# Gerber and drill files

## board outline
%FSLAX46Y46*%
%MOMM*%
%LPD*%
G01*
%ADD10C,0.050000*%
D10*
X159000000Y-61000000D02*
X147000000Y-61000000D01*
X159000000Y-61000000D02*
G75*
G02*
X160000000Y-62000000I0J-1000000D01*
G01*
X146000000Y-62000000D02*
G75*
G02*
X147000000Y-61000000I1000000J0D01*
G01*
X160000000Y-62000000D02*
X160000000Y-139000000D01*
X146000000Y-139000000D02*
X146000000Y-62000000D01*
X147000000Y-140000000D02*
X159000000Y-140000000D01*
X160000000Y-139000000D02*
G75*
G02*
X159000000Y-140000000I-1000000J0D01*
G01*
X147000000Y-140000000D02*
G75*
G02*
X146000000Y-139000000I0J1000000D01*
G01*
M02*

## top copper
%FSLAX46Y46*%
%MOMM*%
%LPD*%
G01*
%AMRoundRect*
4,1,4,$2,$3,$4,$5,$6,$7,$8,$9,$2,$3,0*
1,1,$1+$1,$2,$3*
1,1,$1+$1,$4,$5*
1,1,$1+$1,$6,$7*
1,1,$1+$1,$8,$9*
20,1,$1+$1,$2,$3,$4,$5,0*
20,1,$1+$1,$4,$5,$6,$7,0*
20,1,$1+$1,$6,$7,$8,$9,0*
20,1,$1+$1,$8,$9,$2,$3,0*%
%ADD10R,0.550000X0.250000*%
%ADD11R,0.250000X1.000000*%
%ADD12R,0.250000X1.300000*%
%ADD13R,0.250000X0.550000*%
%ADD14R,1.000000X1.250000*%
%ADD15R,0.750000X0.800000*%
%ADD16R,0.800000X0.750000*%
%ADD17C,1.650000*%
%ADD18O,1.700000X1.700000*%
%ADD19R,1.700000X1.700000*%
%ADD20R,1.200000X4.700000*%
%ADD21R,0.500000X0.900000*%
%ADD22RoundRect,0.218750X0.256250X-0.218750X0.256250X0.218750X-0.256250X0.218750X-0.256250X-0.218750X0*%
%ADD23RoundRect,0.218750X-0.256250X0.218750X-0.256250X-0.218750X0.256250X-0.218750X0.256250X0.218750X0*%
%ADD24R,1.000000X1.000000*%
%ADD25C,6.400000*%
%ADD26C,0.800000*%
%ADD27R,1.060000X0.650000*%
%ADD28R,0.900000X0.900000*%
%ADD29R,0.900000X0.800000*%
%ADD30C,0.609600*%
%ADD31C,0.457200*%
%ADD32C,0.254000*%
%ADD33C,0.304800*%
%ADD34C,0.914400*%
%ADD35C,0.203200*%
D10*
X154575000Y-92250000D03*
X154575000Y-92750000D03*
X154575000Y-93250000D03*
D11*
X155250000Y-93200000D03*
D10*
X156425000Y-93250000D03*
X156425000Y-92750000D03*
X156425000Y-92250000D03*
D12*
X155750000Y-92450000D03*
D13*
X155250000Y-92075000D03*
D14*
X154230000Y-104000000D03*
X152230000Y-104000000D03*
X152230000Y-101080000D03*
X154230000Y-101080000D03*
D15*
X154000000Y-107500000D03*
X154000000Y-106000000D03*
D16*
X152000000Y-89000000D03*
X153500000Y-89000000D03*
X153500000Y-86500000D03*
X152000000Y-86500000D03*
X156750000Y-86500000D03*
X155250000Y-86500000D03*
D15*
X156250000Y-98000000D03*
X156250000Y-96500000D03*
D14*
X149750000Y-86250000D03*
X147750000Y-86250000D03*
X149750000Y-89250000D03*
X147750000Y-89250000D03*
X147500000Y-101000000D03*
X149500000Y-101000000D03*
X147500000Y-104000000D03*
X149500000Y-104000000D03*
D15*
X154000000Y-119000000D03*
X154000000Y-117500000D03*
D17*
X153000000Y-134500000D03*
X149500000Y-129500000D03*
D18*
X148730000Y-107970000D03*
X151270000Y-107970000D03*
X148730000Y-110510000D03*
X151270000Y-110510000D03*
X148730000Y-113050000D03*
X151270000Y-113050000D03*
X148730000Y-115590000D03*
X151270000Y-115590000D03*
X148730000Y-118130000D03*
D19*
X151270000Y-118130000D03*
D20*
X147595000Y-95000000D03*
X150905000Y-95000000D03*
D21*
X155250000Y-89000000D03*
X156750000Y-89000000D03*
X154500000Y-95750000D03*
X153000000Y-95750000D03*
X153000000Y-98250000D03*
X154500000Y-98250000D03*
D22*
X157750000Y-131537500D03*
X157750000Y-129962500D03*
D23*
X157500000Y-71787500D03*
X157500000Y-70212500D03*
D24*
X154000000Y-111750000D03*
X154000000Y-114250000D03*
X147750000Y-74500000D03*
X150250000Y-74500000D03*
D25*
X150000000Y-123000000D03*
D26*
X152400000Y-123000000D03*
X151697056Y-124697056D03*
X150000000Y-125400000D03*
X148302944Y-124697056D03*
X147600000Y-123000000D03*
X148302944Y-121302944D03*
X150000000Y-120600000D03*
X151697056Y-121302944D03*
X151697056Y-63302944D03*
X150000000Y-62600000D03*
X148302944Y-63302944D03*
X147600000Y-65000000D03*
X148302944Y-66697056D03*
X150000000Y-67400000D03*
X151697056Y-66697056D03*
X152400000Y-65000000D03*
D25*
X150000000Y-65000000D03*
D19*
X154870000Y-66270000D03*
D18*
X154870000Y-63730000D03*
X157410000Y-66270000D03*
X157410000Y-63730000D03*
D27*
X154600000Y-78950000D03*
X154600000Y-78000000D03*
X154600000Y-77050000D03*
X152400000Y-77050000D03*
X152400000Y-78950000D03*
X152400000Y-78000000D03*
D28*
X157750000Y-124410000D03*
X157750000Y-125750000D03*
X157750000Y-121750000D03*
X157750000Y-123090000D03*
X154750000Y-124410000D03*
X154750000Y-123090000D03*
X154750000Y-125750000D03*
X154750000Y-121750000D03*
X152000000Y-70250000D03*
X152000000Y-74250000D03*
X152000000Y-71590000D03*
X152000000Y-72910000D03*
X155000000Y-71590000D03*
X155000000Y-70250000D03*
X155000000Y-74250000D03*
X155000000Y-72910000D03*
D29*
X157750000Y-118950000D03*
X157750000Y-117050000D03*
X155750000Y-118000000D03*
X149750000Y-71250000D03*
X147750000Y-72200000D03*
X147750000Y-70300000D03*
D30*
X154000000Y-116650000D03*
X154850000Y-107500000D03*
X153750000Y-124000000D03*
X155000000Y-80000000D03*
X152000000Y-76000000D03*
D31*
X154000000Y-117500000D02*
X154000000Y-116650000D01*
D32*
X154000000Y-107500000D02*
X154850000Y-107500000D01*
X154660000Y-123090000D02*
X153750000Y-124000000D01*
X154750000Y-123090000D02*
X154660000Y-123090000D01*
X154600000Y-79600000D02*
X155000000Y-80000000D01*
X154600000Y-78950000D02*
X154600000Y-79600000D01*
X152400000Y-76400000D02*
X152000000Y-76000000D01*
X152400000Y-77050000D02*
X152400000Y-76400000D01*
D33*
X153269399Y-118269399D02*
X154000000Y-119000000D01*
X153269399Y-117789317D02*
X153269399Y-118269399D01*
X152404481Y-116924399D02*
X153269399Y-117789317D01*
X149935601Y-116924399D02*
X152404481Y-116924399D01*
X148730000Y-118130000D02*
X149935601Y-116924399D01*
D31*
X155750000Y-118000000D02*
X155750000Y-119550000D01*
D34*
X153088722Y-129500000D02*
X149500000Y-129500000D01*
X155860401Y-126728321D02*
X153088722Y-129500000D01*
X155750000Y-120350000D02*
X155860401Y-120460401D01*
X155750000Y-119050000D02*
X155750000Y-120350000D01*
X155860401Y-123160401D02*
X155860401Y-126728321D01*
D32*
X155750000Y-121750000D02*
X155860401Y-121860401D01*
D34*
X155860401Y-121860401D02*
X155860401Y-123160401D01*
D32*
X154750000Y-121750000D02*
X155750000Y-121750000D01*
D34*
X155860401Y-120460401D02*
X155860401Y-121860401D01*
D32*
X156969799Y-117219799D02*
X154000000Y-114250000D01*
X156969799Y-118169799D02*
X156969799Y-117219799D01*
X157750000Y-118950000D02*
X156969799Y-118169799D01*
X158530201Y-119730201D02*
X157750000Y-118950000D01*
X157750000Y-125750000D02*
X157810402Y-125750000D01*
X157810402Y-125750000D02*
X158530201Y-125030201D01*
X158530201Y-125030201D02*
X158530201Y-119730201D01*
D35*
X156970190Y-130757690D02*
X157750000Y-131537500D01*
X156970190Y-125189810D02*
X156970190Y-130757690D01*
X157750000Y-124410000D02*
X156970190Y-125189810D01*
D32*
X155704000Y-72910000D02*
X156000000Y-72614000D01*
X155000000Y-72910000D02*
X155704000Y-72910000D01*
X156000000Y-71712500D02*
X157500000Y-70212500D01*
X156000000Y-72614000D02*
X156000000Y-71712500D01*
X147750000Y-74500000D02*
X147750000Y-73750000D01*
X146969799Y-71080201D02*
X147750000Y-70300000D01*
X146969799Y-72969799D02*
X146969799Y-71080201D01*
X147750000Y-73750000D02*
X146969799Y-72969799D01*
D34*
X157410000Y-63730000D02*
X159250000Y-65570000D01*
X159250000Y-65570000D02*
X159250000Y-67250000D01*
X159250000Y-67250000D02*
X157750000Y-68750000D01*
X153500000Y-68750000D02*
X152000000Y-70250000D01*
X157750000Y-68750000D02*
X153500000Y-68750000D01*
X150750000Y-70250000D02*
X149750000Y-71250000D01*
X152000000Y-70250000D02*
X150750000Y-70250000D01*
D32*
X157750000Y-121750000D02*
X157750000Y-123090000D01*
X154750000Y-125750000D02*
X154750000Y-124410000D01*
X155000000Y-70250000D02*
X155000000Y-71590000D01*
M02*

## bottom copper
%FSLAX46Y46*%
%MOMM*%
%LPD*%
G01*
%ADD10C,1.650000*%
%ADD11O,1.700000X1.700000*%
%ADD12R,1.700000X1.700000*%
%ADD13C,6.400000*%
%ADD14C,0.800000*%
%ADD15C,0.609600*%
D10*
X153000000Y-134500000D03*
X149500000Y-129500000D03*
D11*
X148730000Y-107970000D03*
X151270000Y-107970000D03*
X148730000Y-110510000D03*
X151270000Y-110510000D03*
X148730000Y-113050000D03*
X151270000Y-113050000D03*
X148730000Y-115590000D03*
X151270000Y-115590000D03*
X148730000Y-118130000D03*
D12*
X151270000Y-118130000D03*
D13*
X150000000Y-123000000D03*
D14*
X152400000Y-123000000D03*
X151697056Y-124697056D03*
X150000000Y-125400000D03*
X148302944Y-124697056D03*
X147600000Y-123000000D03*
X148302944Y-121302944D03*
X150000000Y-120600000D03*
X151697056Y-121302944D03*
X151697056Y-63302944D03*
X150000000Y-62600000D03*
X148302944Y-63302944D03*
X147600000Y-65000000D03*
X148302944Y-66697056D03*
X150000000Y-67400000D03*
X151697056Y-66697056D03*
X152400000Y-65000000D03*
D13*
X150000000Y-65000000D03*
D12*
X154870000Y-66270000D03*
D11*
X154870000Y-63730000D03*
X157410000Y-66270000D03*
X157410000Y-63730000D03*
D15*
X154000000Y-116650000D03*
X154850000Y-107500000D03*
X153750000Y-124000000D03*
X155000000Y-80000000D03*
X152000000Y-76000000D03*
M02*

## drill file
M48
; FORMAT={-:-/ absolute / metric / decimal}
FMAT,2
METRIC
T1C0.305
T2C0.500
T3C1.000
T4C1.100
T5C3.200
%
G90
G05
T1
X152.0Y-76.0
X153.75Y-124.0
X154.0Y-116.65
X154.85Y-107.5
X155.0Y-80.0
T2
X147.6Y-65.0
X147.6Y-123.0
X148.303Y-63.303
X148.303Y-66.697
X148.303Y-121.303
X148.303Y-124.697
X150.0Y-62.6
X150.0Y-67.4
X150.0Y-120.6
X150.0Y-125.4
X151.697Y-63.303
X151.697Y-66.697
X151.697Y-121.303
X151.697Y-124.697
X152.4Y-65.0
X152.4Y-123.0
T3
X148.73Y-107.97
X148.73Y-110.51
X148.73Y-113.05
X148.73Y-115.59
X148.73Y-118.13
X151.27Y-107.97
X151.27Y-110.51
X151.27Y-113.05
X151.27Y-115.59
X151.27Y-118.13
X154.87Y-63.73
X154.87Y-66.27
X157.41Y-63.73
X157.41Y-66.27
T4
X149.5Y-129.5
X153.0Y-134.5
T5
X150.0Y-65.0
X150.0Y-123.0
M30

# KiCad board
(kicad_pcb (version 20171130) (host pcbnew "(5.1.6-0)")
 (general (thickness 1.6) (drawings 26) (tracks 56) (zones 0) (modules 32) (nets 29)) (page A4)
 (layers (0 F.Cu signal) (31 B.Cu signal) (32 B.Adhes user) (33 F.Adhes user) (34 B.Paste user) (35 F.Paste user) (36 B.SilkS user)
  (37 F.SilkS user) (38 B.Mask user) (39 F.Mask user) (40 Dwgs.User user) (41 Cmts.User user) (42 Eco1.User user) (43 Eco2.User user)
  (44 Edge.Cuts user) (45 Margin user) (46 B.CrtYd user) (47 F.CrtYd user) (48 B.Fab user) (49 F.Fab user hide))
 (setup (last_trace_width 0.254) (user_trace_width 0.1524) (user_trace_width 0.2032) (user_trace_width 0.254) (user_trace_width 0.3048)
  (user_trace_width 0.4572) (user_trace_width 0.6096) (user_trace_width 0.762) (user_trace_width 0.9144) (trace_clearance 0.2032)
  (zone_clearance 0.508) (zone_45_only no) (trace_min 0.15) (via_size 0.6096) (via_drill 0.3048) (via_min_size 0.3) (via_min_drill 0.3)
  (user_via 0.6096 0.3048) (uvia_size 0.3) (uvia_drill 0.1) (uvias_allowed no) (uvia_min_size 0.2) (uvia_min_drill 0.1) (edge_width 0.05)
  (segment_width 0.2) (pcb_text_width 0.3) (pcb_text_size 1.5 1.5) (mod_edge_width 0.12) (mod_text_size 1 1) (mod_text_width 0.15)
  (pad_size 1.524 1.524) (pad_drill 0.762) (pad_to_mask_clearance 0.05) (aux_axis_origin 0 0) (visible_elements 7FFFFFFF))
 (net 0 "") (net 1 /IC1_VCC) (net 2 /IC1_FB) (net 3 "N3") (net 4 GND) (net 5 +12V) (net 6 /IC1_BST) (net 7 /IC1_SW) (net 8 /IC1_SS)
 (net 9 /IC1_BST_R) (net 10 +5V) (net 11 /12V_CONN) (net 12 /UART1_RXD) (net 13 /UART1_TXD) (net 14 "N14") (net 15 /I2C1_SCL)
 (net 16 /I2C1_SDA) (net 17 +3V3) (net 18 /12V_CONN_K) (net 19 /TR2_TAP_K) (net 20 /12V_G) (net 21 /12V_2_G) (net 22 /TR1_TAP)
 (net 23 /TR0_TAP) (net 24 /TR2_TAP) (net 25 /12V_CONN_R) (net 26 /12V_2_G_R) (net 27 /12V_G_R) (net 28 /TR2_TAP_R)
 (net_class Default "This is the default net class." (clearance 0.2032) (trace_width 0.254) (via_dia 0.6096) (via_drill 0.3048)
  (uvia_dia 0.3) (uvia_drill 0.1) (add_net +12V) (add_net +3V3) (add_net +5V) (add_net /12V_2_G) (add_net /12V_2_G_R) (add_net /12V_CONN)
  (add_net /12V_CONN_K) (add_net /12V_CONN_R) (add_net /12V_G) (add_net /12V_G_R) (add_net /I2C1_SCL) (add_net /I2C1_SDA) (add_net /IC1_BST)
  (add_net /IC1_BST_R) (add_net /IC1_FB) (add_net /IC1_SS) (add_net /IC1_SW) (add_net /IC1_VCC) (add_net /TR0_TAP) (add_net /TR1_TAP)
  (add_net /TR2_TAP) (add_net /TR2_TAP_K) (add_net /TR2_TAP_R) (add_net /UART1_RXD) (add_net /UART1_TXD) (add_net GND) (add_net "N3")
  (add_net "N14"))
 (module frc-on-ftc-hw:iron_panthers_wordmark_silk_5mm (layer F.Cu) (at 157.5 108 90)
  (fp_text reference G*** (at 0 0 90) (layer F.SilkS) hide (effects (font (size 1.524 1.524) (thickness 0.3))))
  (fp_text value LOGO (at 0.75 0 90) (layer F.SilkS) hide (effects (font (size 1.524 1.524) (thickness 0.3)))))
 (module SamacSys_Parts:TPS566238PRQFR (layer F.Cu) (at 155.5 92.75)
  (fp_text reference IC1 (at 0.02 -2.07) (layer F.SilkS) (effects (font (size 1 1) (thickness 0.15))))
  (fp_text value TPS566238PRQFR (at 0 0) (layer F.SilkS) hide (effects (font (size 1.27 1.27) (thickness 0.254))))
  (pad 1 smd rect (at -0.925 -0.5 90) (size 0.25 0.55) (layers F.Cu F.Paste F.Mask) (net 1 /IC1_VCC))
  (pad 2 smd rect (at -0.925 0 90) (size 0.25 0.55) (layers F.Cu F.Paste F.Mask) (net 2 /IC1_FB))
  (pad 3 smd rect (at -0.925 0.5 90) (size 0.25 0.55) (layers F.Cu F.Paste F.Mask) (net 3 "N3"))
  (pad 4 smd rect (at -0.25 0.45) (size 0.25 1) (layers F.Cu F.Paste F.Mask) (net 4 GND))
  (pad 5 smd rect (at 0.925 0.5 90) (size 0.25 0.55) (layers F.Cu F.Paste F.Mask) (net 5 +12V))
  (pad 6 smd rect (at 0.925 0 90) (size 0.25 0.55) (layers F.Cu F.Paste F.Mask) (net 5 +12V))
  (pad 7 smd rect (at 0.925 -0.5 90) (size 0.25 0.55) (layers F.Cu F.Paste F.Mask) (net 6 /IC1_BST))
  (pad 8 smd rect (at 0.25 -0.3) (size 0.25 1.3) (layers F.Cu F.Paste F.Mask) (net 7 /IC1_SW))
  (pad 9 smd rect (at -0.25 -0.675) (size 0.25 0.55) (layers F.Cu F.Paste F.Mask) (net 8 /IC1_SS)))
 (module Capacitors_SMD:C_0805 (layer F.Cu) (at 153.23 104 180)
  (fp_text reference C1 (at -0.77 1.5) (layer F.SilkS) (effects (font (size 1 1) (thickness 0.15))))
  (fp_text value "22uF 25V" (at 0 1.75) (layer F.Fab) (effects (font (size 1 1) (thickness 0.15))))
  (pad 1 smd rect (at -1 0 180) (size 1 1.25) (layers F.Cu F.Paste F.Mask) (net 5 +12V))
  (pad 2 smd rect (at 1 0 180) (size 1 1.25) (layers F.Cu F.Paste F.Mask) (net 4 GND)))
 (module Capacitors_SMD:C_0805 (layer F.Cu) (at 153.23 101.08 180)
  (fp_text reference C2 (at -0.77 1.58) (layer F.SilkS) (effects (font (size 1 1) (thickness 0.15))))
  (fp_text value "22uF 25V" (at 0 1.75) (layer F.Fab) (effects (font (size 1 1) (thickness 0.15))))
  (pad 2 smd rect (at 1 0 180) (size 1 1.25) (layers F.Cu F.Paste F.Mask) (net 4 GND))
  (pad 1 smd rect (at -1 0 180) (size 1 1.25) (layers F.Cu F.Paste F.Mask) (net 5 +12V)))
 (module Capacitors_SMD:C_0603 (layer F.Cu) (at 154 106.75 270)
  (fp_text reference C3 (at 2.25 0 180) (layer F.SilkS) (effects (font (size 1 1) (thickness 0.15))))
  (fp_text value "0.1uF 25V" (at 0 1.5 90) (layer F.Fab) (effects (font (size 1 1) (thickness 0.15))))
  (pad 2 smd rect (at 0.75 0 270) (size 0.8 0.75) (layers F.Cu F.Paste F.Mask) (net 4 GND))
  (pad 1 smd rect (at -0.75 0 270) (size 0.8 0.75) (layers F.Cu F.Paste F.Mask) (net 5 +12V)))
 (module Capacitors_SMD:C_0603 (layer F.Cu) (at 152.75 89 180)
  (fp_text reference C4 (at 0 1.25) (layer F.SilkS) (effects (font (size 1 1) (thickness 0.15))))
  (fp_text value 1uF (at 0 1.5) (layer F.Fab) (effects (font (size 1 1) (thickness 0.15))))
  (pad 2 smd rect (at 0.75 0 180) (size 0.8 0.75) (layers F.Cu F.Paste F.Mask) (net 4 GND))
  (pad 1 smd rect (at -0.75 0 180) (size 0.8 0.75) (layers F.Cu F.Paste F.Mask) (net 1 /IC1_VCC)))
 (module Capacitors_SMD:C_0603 (layer F.Cu) (at 152.75 86.5 180)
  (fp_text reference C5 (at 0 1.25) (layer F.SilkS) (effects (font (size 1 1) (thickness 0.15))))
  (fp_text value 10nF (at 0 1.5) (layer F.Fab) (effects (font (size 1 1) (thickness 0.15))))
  (pad 1 smd rect (at -0.75 0 180) (size 0.8 0.75) (layers F.Cu F.Paste F.Mask) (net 8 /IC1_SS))
  (pad 2 smd rect (at 0.75 0 180) (size 0.8 0.75) (layers F.Cu F.Paste F.Mask) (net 4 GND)))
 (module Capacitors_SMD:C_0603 (layer F.Cu) (at 156 86.5)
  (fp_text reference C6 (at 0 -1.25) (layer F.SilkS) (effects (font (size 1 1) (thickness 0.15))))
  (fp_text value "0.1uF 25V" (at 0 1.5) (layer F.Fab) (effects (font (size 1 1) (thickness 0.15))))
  (pad 2 smd rect (at 0.75 0) (size 0.8 0.75) (layers F.Cu F.Paste F.Mask) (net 7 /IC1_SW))
  (pad 1 smd rect (at -0.75 0) (size 0.8 0.75) (layers F.Cu F.Paste F.Mask) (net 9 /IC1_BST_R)))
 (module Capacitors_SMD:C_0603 (layer F.Cu) (at 156.25 97.25 90)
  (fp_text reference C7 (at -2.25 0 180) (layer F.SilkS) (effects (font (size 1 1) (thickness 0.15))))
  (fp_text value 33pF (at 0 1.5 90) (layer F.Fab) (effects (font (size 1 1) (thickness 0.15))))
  (pad 1 smd rect (at -0.75 0 90) (size 0.8 0.75) (layers F.Cu F.Paste F.Mask) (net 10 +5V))
  (pad 2 smd rect (at 0.75 0 90) (size 0.8 0.75) (layers F.Cu F.Paste F.Mask) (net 2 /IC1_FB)))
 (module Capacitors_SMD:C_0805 (layer F.Cu) (at 148.75 86.25)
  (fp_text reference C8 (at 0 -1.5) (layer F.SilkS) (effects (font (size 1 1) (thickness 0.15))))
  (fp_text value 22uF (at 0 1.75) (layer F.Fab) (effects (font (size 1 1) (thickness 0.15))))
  (pad 2 smd rect (at 1 0) (size 1 1.25) (layers F.Cu F.Paste F.Mask) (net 4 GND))
  (pad 1 smd rect (at -1 0) (size 1 1.25) (layers F.Cu F.Paste F.Mask) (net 10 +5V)))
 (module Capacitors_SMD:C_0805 (layer F.Cu) (at 148.75 89.25)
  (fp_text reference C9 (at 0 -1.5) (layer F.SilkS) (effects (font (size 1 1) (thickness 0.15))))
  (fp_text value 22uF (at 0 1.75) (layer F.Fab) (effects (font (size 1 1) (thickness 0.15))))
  (pad 2 smd rect (at 1 0) (size 1 1.25) (layers F.Cu F.Paste F.Mask) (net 4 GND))
  (pad 1 smd rect (at -1 0) (size 1 1.25) (layers F.Cu F.Paste F.Mask) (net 10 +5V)))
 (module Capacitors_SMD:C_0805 (layer F.Cu) (at 148.5 101)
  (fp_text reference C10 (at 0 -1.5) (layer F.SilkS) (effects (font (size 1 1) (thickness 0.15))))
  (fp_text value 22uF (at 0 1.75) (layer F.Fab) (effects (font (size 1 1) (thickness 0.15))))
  (pad 1 smd rect (at -1 0) (size 1 1.25) (layers F.Cu F.Paste F.Mask) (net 10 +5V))
  (pad 2 smd rect (at 1 0) (size 1 1.25) (layers F.Cu F.Paste F.Mask) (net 4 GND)))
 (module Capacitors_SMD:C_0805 (layer F.Cu) (at 148.5 104)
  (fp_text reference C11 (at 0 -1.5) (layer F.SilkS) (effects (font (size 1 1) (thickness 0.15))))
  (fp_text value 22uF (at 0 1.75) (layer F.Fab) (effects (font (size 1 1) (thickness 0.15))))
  (pad 1 smd rect (at -1 0) (size 1 1.25) (layers F.Cu F.Paste F.Mask) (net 10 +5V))
  (pad 2 smd rect (at 1 0) (size 1 1.25) (layers F.Cu F.Paste F.Mask) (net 4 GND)))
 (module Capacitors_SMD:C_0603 (layer F.Cu) (at 154 118.25 90)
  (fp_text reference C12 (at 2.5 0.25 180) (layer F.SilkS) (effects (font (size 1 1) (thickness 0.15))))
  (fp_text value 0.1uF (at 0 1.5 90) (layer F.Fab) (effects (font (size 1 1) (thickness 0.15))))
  (pad 1 smd rect (at -0.75 0 90) (size 0.8 0.75) (layers F.Cu F.Paste F.Mask) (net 10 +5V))
  (pad 2 smd rect (at 0.75 0 90) (size 0.8 0.75) (layers F.Cu F.Paste F.Mask) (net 4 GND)))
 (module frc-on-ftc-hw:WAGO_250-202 (layer F.Cu) (at 153 134.5 180)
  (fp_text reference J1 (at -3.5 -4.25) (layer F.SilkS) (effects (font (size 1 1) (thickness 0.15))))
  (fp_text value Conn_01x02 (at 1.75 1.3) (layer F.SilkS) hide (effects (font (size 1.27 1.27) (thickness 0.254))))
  (pad 1 thru_hole circle (at 0 0 180) (size 1.65 1.65) (drill 1.1) (layers *.Cu *.Mask) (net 4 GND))
  (pad 2 thru_hole circle (at 3.5 5 180) (size 1.65 1.65) (drill 1.1) (layers *.Cu *.Mask) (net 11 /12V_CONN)))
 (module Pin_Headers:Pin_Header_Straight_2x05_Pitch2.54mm (layer F.Cu) (at 151.27 118.13 180)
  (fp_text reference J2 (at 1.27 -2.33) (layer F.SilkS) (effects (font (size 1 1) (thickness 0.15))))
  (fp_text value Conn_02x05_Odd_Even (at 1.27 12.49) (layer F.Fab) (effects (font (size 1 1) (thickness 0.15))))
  (pad 10 thru_hole oval (at 2.54 10.16 180) (size 1.7 1.7) (drill 1) (layers *.Cu *.Mask) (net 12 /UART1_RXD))
  (pad 9 thru_hole oval (at 0 10.16 180) (size 1.7 1.7) (drill 1) (layers *.Cu *.Mask) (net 4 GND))
  (pad 8 thru_hole oval (at 2.54 7.62 180) (size 1.7 1.7) (drill 1) (layers *.Cu *.Mask) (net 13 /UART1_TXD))
  (pad 7 thru_hole oval (at 0 7.62 180) (size 1.7 1.7) (drill 1) (layers *.Cu *.Mask) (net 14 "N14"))
  (pad 6 thru_hole oval (at 2.54 5.08 180) (size 1.7 1.7) (drill 1) (layers *.Cu *.Mask) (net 4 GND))
  (pad 5 thru_hole oval (at 0 5.08 180) (size 1.7 1.7) (drill 1) (layers *.Cu *.Mask) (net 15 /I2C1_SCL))
  (pad 4 thru_hole oval (at 2.54 2.54 180) (size 1.7 1.7) (drill 1) (layers *.Cu *.Mask) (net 10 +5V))
  (pad 3 thru_hole oval (at 0 2.54 180) (size 1.7 1.7) (drill 1) (layers *.Cu *.Mask) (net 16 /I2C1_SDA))
  (pad 2 thru_hole oval (at 2.54 0 180) (size 1.7 1.7) (drill 1) (layers *.Cu *.Mask) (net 10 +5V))
  (pad 1 thru_hole rect (at 0 0 180) (size 1.7 1.7) (drill 1) (layers *.Cu *.Mask) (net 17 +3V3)))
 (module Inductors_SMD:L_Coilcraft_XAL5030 (layer F.Cu) (at 149.25 95 180)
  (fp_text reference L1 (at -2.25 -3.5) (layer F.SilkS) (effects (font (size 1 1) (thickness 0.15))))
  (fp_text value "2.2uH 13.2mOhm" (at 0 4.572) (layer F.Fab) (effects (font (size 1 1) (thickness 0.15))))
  (pad 2 smd rect (at 1.655 0 180) (size 1.2 4.7) (layers F.Cu F.Paste F.Mask) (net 10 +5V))
  (pad 1 smd rect (at -1.655 0 180) (size 1.2 4.7) (layers F.Cu F.Paste F.Mask) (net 7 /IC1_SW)))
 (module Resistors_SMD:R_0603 (layer F.Cu) (at 156 89)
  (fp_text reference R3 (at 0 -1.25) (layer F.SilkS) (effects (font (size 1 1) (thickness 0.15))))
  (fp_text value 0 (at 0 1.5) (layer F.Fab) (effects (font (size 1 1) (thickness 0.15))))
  (pad 1 smd rect (at -0.75 0) (size 0.5 0.9) (layers F.Cu F.Paste F.Mask) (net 9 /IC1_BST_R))
  (pad 2 smd rect (at 0.75 0) (size 0.5 0.9) (layers F.Cu F.Paste F.Mask) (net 6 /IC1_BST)))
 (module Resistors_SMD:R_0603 (layer F.Cu) (at 153.75 95.75)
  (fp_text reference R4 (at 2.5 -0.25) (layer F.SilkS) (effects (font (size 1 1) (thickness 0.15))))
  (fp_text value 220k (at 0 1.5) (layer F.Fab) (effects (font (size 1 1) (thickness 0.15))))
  (pad 2 smd rect (at 0.75 0) (size 0.5 0.9) (layers F.Cu F.Paste F.Mask) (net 2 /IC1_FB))
  (pad 1 smd rect (at -0.75 0) (size 0.5 0.9) (layers F.Cu F.Paste F.Mask) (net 10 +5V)))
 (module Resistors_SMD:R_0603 (layer F.Cu) (at 153.75 98.25 180)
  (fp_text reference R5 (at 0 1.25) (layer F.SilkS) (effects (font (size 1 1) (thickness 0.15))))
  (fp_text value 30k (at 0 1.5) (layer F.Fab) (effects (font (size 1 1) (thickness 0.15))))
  (pad 2 smd rect (at 0.75 0 180) (size 0.5 0.9) (layers F.Cu F.Paste F.Mask) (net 4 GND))
  (pad 1 smd rect (at -0.75 0 180) (size 0.5 0.9) (layers F.Cu F.Paste F.Mask) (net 2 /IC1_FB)))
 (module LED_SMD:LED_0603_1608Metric (layer F.Cu) (at 157.75 130.75 90)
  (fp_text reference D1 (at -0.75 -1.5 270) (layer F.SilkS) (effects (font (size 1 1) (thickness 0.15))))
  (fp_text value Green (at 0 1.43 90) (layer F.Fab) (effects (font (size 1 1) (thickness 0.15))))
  (pad 1 smd roundrect (at -0.7875 0 90) (size 0.875 0.95) (layers F.Cu F.Paste F.Mask) (roundrect_rratio 0.25) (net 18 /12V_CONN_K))
  (pad 2 smd roundrect (at 0.7875 0 90) (size 0.875 0.95) (layers F.Cu F.Paste F.Mask) (roundrect_rratio 0.25) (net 5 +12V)))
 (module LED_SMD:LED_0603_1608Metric (layer F.Cu) (at 157.5 71 270)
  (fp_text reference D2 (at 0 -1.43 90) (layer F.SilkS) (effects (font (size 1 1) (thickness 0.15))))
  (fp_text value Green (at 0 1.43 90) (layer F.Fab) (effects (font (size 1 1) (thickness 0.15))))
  (pad 2 smd roundrect (at 0.7875 0 270) (size 0.875 0.95) (layers F.Cu F.Paste F.Mask) (roundrect_rratio 0.25) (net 5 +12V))
  (pad 1 smd roundrect (at -0.7875 0 270) (size 0.875 0.95) (layers F.Cu F.Paste F.Mask) (roundrect_rratio 0.25) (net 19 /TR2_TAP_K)))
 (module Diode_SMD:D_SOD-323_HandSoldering (layer F.Cu) (at 154 113 270)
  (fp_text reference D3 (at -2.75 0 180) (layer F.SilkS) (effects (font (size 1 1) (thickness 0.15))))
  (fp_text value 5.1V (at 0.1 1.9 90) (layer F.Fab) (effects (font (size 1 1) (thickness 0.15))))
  (pad 1 smd rect (at -1.25 0 270) (size 1 1) (layers F.Cu F.Paste F.Mask) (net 5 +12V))
  (pad 2 smd rect (at 1.25 0 270) (size 1 1) (layers F.Cu F.Paste F.Mask) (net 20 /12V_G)))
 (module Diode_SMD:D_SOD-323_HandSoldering (layer F.Cu) (at 149 74.5 180)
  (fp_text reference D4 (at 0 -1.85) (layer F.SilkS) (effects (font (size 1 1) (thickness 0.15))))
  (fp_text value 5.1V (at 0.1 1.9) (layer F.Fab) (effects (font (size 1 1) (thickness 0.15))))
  (pad 2 smd rect (at 1.25 0 180) (size 1 1) (layers F.Cu F.Paste F.Mask) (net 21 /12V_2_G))
  (pad 1 smd rect (at -1.25 0 180) (size 1 1) (layers F.Cu F.Paste F.Mask) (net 5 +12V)))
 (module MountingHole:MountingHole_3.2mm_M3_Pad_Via (layer F.Cu) (at 150 123)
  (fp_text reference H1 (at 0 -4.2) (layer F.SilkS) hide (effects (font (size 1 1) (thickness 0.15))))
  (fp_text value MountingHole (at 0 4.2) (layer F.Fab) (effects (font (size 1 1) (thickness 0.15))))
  (pad 1 thru_hole circle (at 0 0) (size 6.4 6.4) (drill 3.2) (layers *.Cu *.Mask))
  (pad 1 thru_hole circle (at 2.4 0) (size 0.8 0.8) (drill 0.5) (layers *.Cu *.Mask))
  (pad 1 thru_hole circle (at 1.697056 1.697056) (size 0.8 0.8) (drill 0.5) (layers *.Cu *.Mask))
  (pad 1 thru_hole circle (at 0 2.4) (size 0.8 0.8) (drill 0.5) (layers *.Cu *.Mask))
  (pad 1 thru_hole circle (at -1.697056 1.697056) (size 0.8 0.8) (drill 0.5) (layers *.Cu *.Mask))
  (pad 1 thru_hole circle (at -2.4 0) (size 0.8 0.8) (drill 0.5) (layers *.Cu *.Mask))
  (pad 1 thru_hole circle (at -1.697056 -1.697056) (size 0.8 0.8) (drill 0.5) (layers *.Cu *.Mask))
  (pad 1 thru_hole circle (at 0 -2.4) (size 0.8 0.8) (drill 0.5) (layers *.Cu *.Mask))
  (pad 1 thru_hole circle (at 1.697056 -1.697056) (size 0.8 0.8) (drill 0.5) (layers *.Cu *.Mask)))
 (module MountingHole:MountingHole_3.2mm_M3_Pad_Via (layer F.Cu) (at 150 65)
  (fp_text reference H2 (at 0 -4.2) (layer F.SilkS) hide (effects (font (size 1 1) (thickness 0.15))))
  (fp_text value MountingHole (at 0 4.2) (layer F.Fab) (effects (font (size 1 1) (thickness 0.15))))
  (pad 1 thru_hole circle (at 1.697056 -1.697056) (size 0.8 0.8) (drill 0.5) (layers *.Cu *.Mask))
  (pad 1 thru_hole circle (at 0 -2.4) (size 0.8 0.8) (drill 0.5) (layers *.Cu *.Mask))
  (pad 1 thru_hole circle (at -1.697056 -1.697056) (size 0.8 0.8) (drill 0.5) (layers *.Cu *.Mask))
  (pad 1 thru_hole circle (at -2.4 0) (size 0.8 0.8) (drill 0.5) (layers *.Cu *.Mask))
  (pad 1 thru_hole circle (at -1.697056 1.697056) (size 0.8 0.8) (drill 0.5) (layers *.Cu *.Mask))
  (pad 1 thru_hole circle (at 0 2.4) (size 0.8 0.8) (drill 0.5) (layers *.Cu *.Mask))
  (pad 1 thru_hole circle (at 1.697056 1.697056) (size 0.8 0.8) (drill 0.5) (layers *.Cu *.Mask))
  (pad 1 thru_hole circle (at 2.4 0) (size 0.8 0.8) (drill 0.5) (layers *.Cu *.Mask))
  (pad 1 thru_hole circle (at 0 0) (size 6.4 6.4) (drill 3.2) (layers *.Cu *.Mask)))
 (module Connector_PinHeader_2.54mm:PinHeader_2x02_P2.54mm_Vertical (layer F.Cu) (at 154.87 66.27 90)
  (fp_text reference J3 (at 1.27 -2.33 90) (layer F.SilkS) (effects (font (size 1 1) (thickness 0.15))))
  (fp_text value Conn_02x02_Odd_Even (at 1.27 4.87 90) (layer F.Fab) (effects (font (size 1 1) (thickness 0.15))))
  (pad 1 thru_hole rect (at 0 0 90) (size 1.7 1.7) (drill 1) (layers *.Cu *.Mask) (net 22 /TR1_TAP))
  (pad 2 thru_hole oval (at 2.54 0 90) (size 1.7 1.7) (drill 1) (layers *.Cu *.Mask) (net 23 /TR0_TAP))
  (pad 3 thru_hole oval (at 0 2.54 90) (size 1.7 1.7) (drill 1) (layers *.Cu *.Mask) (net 4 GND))
  (pad 4 thru_hole oval (at 2.54 2.54 90) (size 1.7 1.7) (drill 1) (layers *.Cu *.Mask) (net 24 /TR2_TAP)))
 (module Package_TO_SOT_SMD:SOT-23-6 (layer F.Cu) (at 153.5 78 180)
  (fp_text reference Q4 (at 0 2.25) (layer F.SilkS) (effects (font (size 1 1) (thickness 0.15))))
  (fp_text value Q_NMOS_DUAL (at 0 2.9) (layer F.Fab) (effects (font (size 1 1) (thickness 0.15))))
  (pad 1 smd rect (at -1.1 -0.95 180) (size 1.06 0.65) (layers F.Cu F.Paste F.Mask) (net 4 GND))
  (pad 2 smd rect (at -1.1 0 180) (size 1.06 0.65) (layers F.Cu F.Paste F.Mask) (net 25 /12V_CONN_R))
  (pad 3 smd rect (at -1.1 0.95 180) (size 1.06 0.65) (layers F.Cu F.Paste F.Mask) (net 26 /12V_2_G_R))
  (pad 4 smd rect (at 1.1 0.95 180) (size 1.06 0.65) (layers F.Cu F.Paste F.Mask) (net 4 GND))
  (pad 6 smd rect (at 1.1 -0.95 180) (size 1.06 0.65) (layers F.Cu F.Paste F.Mask) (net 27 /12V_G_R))
  (pad 5 smd rect (at 1.1 0 180) (size 1.06 0.65) (layers F.Cu F.Paste F.Mask) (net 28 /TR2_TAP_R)))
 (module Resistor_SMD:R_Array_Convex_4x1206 (layer F.Cu) (at 156.25 123.75)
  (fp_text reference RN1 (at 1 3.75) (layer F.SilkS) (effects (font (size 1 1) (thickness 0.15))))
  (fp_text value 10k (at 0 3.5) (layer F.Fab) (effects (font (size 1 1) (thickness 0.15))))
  (pad 6 smd rect (at 1.5 0.66) (size 0.9 0.9) (layers F.Cu F.Paste F.Mask) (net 18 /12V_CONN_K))
  (pad 5 smd rect (at 1.5 2) (size 0.9 0.9) (layers F.Cu F.Paste F.Mask) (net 20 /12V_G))
  (pad 8 smd rect (at 1.5 -2) (size 0.9 0.9) (layers F.Cu F.Paste F.Mask) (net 25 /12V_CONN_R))
  (pad 7 smd rect (at 1.5 -0.66) (size 0.9 0.9) (layers F.Cu F.Paste F.Mask) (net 25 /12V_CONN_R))
  (pad 3 smd rect (at -1.5 0.66) (size 0.9 0.9) (layers F.Cu F.Paste F.Mask) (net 27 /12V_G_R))
  (pad 2 smd rect (at -1.5 -0.66) (size 0.9 0.9) (layers F.Cu F.Paste F.Mask) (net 4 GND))
  (pad 4 smd rect (at -1.5 2) (size 0.9 0.9) (layers F.Cu F.Paste F.Mask) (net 27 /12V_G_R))
  (pad 1 smd rect (at -1.5 -2) (size 0.9 0.9) (layers F.Cu F.Paste F.Mask) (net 11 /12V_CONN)))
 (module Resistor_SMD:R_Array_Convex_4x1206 (layer F.Cu) (at 153.5 72.25)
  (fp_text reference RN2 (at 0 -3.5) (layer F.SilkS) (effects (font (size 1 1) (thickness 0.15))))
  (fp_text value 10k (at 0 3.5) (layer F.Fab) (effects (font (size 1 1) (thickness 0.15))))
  (pad 1 smd rect (at -1.5 -2) (size 0.9 0.9) (layers F.Cu F.Paste F.Mask) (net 24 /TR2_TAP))
  (pad 4 smd rect (at -1.5 2) (size 0.9 0.9) (layers F.Cu F.Paste F.Mask) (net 26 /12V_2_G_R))
  (pad 2 smd rect (at -1.5 -0.66) (size 0.9 0.9) (layers F.Cu F.Paste F.Mask) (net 4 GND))
  (pad 3 smd rect (at -1.5 0.66) (size 0.9 0.9) (layers F.Cu F.Paste F.Mask) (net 26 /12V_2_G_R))
  (pad 7 smd rect (at 1.5 -0.66) (size 0.9 0.9) (layers F.Cu F.Paste F.Mask) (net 28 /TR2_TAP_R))
  (pad 8 smd rect (at 1.5 -2) (size 0.9 0.9) (layers F.Cu F.Paste F.Mask) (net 28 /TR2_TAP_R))
  (pad 5 smd rect (at 1.5 2) (size 0.9 0.9) (layers F.Cu F.Paste F.Mask) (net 21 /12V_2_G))
  (pad 6 smd rect (at 1.5 0.66) (size 0.9 0.9) (layers F.Cu F.Paste F.Mask) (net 19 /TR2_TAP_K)))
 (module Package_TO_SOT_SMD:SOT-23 (layer F.Cu) (at 156.75 118 180)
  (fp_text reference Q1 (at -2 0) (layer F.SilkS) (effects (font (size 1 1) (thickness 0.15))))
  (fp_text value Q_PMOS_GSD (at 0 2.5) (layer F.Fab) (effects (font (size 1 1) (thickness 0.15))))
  (pad 1 smd rect (at -1 -0.95 180) (size 0.9 0.8) (layers F.Cu F.Paste F.Mask) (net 20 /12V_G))
  (pad 2 smd rect (at -1 0.95 180) (size 0.9 0.8) (layers F.Cu F.Paste F.Mask) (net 5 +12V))
  (pad 3 smd rect (at 1 0 180) (size 0.9 0.8) (layers F.Cu F.Paste F.Mask) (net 11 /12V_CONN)))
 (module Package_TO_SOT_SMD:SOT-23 (layer F.Cu) (at 148.75 71.25)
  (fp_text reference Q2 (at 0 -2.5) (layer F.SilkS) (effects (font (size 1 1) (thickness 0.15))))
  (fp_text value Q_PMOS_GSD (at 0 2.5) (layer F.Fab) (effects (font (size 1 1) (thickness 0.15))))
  (pad 3 smd rect (at 1 0) (size 0.9 0.8) (layers F.Cu F.Paste F.Mask) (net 24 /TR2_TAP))
  (pad 2 smd rect (at -1 0.95) (size 0.9 0.8) (layers F.Cu F.Paste F.Mask) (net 5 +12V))
  (pad 1 smd rect (at -1 -0.95) (size 0.9 0.8) (layers F.Cu F.Paste F.Mask) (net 21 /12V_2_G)))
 (gr_line (start 159 61) (end 147 61) (layer Edge.Cuts) (width 0.05))
 (gr_arc (start 159 62) (end 160 62) (angle -90) (layer Edge.Cuts) (width 0.05))
 (gr_arc (start 147 62) (end 147 61) (angle -90) (layer Edge.Cuts) (width 0.05))
 (gr_line (start 160 62) (end 160 139) (layer Edge.Cuts) (width 0.05))
 (gr_line (start 146 139) (end 146 62) (layer Edge.Cuts) (width 0.05))
 (gr_line (start 147 140) (end 159 140) (layer Edge.Cuts) (width 0.05))
 (gr_arc (start 159 139) (end 159 140) (angle -90) (layer Edge.Cuts) (width 0.05))
 (gr_arc (start 147 139) (end 146 139) (angle -90) (layer Edge.Cuts) (width 0.05))
 (via (at 154 116.65) (size 0.6096) (drill 0.3048) (layers F.Cu B.Cu) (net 4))
 (segment (start 154 117.5) (end 154 116.65) (width 0.4572) (layer F.Cu) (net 4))
 (via (at 154.85 107.5) (size 0.6096) (drill 0.3048) (layers F.Cu B.Cu) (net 4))
 (segment (start 154 107.5) (end 154.85 107.5) (width 0.254) (layer F.Cu) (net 4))
 (via (at 153.75 124) (size 0.6096) (drill 0.3048) (layers F.Cu B.Cu) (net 4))
 (segment (start 154.66 123.09) (end 153.75 124) (width 0.254) (layer F.Cu) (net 4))
 (segment (start 154.75 123.09) (end 154.66 123.09) (width 0.254) (layer F.Cu) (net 4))
 (segment (start 154.6 79.6) (end 155 80) (width 0.254) (layer F.Cu) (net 4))
 (via (at 155 80) (size 0.6096) (drill 0.3048) (layers F.Cu B.Cu) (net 4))
 (segment (start 154.6 78.95) (end 154.6 79.6) (width 0.254) (layer F.Cu) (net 4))
 (via (at 152 76) (size 0.6096) (drill 0.3048) (layers F.Cu B.Cu) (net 4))
 (segment (start 152.4 76.4) (end 152 76) (width 0.254) (layer F.Cu) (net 4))
 (segment (start 152.4 77.05) (end 152.4 76.4) (width 0.254) (layer F.Cu) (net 4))
 (segment (start 153.269399 118.269399) (end 154 119) (width 0.3048) (layer F.Cu) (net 10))
 (segment (start 153.269399 117.789317) (end 153.269399 118.269399) (width 0.3048) (layer F.Cu) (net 10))
 (segment (start 152.404481 116.924399) (end 153.269399 117.789317) (width 0.3048) (layer F.Cu) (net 10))
 (segment (start 149.935601 116.924399) (end 152.404481 116.924399) (width 0.3048) (layer F.Cu) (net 10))
 (segment (start 148.73 118.13) (end 149.935601 116.924399) (width 0.3048) (layer F.Cu) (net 10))
 (segment (start 155.75 118) (end 155.75 119.55) (width 0.4572) (layer F.Cu) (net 11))
 (segment (start 153.088722 129.5) (end 149.5 129.5) (width 0.9144) (layer F.Cu) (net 11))
 (segment (start 155.860401 126.728321) (end 153.088722 129.5) (width 0.9144) (layer F.Cu) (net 11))
 (segment (start 155.75 120.35) (end 155.860401 120.460401) (width 0.9144) (layer F.Cu) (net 11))
 (segment (start 155.75 119.05) (end 155.75 120.35) (width 0.9144) (layer F.Cu) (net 11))
 (segment (start 155.860401 123.160401) (end 155.860401 126.728321) (width 0.9144) (layer F.Cu) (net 11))
 (segment (start 155.75 121.75) (end 155.860401 121.860401) (width 0.254) (layer F.Cu) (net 11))
 (segment (start 155.860401 121.860401) (end 155.860401 123.160401) (width 0.9144) (layer F.Cu) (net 11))
 (segment (start 154.75 121.75) (end 155.75 121.75) (width 0.254) (layer F.Cu) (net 11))
 (segment (start 155.860401 120.460401) (end 155.860401 121.860401) (width 0.9144) (layer F.Cu) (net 11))
 (segment (start 156.969799 117.219799) (end 154 114.25) (width 0.254) (layer F.Cu) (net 20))
 (segment (start 156.969799 118.169799) (end 156.969799 117.219799) (width 0.254) (layer F.Cu) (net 20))
 (segment (start 157.75 118.95) (end 156.969799 118.169799) (width 0.254) (layer F.Cu) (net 20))
 (segment (start 158.530201 119.730201) (end 157.75 118.95) (width 0.254) (layer F.Cu) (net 20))
 (segment (start 157.75 125.75) (end 157.810402 125.75) (width 0.254) (layer F.Cu) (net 20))
 (segment (start 157.810402 125.75) (end 158.530201 125.030201) (width 0.254) (layer F.Cu) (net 20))
 (segment (start 158.530201 125.030201) (end 158.530201 119.730201) (width 0.254) (layer F.Cu) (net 20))
 (segment (start 156.97019 130.75769) (end 157.75 131.5375) (width 0.2032) (layer F.Cu) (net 18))
 (segment (start 156.97019 125.18981) (end 156.97019 130.75769) (width 0.2032) (layer F.Cu) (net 18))
 (segment (start 157.75 124.41) (end 156.97019 125.18981) (width 0.2032) (layer F.Cu) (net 18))
 (segment (start 155.704 72.91) (end 156 72.614) (width 0.254) (layer F.Cu) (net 19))
 (segment (start 155 72.91) (end 155.704 72.91) (width 0.254) (layer F.Cu) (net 19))
 (segment (start 156 71.7125) (end 157.5 70.2125) (width 0.254) (layer F.Cu) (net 19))
 (segment (start 156 72.614) (end 156 71.7125) (width 0.254) (layer F.Cu) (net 19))
 (segment (start 147.75 74.5) (end 147.75 73.75) (width 0.254) (layer F.Cu) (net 21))
 (segment (start 146.969799 71.080201) (end 147.75 70.3) (width 0.254) (layer F.Cu) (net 21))
 (segment (start 146.969799 72.969799) (end 146.969799 71.080201) (width 0.254) (layer F.Cu) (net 21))
 (segment (start 147.75 73.75) (end 146.969799 72.969799) (width 0.254) (layer F.Cu) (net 21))
 (segment (start 157.41 63.73) (end 159.25 65.57) (width 0.9144) (layer F.Cu) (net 24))
 (segment (start 159.25 65.57) (end 159.25 67.25) (width 0.9144) (layer F.Cu) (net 24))
 (segment (start 159.25 67.25) (end 157.75 68.75) (width 0.9144) (layer F.Cu) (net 24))
 (segment (start 153.5 68.75) (end 152 70.25) (width 0.9144) (layer F.Cu) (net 24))
 (segment (start 157.75 68.75) (end 153.5 68.75) (width 0.9144) (layer F.Cu) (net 24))
 (segment (start 150.75 70.25) (end 149.75 71.25) (width 0.9144) (layer F.Cu) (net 24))
 (segment (start 152 70.25) (end 150.75 70.25) (width 0.9144) (layer F.Cu) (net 24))
 (segment (start 157.75 121.75) (end 157.75 123.09) (width 0.254) (layer F.Cu) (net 25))
 (segment (start 154.75 125.75) (end 154.75 124.41) (width 0.254) (layer F.Cu) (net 27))
 (segment (start 155 70.25) (end 155 71.59) (width 0.254) (layer F.Cu) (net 28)))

